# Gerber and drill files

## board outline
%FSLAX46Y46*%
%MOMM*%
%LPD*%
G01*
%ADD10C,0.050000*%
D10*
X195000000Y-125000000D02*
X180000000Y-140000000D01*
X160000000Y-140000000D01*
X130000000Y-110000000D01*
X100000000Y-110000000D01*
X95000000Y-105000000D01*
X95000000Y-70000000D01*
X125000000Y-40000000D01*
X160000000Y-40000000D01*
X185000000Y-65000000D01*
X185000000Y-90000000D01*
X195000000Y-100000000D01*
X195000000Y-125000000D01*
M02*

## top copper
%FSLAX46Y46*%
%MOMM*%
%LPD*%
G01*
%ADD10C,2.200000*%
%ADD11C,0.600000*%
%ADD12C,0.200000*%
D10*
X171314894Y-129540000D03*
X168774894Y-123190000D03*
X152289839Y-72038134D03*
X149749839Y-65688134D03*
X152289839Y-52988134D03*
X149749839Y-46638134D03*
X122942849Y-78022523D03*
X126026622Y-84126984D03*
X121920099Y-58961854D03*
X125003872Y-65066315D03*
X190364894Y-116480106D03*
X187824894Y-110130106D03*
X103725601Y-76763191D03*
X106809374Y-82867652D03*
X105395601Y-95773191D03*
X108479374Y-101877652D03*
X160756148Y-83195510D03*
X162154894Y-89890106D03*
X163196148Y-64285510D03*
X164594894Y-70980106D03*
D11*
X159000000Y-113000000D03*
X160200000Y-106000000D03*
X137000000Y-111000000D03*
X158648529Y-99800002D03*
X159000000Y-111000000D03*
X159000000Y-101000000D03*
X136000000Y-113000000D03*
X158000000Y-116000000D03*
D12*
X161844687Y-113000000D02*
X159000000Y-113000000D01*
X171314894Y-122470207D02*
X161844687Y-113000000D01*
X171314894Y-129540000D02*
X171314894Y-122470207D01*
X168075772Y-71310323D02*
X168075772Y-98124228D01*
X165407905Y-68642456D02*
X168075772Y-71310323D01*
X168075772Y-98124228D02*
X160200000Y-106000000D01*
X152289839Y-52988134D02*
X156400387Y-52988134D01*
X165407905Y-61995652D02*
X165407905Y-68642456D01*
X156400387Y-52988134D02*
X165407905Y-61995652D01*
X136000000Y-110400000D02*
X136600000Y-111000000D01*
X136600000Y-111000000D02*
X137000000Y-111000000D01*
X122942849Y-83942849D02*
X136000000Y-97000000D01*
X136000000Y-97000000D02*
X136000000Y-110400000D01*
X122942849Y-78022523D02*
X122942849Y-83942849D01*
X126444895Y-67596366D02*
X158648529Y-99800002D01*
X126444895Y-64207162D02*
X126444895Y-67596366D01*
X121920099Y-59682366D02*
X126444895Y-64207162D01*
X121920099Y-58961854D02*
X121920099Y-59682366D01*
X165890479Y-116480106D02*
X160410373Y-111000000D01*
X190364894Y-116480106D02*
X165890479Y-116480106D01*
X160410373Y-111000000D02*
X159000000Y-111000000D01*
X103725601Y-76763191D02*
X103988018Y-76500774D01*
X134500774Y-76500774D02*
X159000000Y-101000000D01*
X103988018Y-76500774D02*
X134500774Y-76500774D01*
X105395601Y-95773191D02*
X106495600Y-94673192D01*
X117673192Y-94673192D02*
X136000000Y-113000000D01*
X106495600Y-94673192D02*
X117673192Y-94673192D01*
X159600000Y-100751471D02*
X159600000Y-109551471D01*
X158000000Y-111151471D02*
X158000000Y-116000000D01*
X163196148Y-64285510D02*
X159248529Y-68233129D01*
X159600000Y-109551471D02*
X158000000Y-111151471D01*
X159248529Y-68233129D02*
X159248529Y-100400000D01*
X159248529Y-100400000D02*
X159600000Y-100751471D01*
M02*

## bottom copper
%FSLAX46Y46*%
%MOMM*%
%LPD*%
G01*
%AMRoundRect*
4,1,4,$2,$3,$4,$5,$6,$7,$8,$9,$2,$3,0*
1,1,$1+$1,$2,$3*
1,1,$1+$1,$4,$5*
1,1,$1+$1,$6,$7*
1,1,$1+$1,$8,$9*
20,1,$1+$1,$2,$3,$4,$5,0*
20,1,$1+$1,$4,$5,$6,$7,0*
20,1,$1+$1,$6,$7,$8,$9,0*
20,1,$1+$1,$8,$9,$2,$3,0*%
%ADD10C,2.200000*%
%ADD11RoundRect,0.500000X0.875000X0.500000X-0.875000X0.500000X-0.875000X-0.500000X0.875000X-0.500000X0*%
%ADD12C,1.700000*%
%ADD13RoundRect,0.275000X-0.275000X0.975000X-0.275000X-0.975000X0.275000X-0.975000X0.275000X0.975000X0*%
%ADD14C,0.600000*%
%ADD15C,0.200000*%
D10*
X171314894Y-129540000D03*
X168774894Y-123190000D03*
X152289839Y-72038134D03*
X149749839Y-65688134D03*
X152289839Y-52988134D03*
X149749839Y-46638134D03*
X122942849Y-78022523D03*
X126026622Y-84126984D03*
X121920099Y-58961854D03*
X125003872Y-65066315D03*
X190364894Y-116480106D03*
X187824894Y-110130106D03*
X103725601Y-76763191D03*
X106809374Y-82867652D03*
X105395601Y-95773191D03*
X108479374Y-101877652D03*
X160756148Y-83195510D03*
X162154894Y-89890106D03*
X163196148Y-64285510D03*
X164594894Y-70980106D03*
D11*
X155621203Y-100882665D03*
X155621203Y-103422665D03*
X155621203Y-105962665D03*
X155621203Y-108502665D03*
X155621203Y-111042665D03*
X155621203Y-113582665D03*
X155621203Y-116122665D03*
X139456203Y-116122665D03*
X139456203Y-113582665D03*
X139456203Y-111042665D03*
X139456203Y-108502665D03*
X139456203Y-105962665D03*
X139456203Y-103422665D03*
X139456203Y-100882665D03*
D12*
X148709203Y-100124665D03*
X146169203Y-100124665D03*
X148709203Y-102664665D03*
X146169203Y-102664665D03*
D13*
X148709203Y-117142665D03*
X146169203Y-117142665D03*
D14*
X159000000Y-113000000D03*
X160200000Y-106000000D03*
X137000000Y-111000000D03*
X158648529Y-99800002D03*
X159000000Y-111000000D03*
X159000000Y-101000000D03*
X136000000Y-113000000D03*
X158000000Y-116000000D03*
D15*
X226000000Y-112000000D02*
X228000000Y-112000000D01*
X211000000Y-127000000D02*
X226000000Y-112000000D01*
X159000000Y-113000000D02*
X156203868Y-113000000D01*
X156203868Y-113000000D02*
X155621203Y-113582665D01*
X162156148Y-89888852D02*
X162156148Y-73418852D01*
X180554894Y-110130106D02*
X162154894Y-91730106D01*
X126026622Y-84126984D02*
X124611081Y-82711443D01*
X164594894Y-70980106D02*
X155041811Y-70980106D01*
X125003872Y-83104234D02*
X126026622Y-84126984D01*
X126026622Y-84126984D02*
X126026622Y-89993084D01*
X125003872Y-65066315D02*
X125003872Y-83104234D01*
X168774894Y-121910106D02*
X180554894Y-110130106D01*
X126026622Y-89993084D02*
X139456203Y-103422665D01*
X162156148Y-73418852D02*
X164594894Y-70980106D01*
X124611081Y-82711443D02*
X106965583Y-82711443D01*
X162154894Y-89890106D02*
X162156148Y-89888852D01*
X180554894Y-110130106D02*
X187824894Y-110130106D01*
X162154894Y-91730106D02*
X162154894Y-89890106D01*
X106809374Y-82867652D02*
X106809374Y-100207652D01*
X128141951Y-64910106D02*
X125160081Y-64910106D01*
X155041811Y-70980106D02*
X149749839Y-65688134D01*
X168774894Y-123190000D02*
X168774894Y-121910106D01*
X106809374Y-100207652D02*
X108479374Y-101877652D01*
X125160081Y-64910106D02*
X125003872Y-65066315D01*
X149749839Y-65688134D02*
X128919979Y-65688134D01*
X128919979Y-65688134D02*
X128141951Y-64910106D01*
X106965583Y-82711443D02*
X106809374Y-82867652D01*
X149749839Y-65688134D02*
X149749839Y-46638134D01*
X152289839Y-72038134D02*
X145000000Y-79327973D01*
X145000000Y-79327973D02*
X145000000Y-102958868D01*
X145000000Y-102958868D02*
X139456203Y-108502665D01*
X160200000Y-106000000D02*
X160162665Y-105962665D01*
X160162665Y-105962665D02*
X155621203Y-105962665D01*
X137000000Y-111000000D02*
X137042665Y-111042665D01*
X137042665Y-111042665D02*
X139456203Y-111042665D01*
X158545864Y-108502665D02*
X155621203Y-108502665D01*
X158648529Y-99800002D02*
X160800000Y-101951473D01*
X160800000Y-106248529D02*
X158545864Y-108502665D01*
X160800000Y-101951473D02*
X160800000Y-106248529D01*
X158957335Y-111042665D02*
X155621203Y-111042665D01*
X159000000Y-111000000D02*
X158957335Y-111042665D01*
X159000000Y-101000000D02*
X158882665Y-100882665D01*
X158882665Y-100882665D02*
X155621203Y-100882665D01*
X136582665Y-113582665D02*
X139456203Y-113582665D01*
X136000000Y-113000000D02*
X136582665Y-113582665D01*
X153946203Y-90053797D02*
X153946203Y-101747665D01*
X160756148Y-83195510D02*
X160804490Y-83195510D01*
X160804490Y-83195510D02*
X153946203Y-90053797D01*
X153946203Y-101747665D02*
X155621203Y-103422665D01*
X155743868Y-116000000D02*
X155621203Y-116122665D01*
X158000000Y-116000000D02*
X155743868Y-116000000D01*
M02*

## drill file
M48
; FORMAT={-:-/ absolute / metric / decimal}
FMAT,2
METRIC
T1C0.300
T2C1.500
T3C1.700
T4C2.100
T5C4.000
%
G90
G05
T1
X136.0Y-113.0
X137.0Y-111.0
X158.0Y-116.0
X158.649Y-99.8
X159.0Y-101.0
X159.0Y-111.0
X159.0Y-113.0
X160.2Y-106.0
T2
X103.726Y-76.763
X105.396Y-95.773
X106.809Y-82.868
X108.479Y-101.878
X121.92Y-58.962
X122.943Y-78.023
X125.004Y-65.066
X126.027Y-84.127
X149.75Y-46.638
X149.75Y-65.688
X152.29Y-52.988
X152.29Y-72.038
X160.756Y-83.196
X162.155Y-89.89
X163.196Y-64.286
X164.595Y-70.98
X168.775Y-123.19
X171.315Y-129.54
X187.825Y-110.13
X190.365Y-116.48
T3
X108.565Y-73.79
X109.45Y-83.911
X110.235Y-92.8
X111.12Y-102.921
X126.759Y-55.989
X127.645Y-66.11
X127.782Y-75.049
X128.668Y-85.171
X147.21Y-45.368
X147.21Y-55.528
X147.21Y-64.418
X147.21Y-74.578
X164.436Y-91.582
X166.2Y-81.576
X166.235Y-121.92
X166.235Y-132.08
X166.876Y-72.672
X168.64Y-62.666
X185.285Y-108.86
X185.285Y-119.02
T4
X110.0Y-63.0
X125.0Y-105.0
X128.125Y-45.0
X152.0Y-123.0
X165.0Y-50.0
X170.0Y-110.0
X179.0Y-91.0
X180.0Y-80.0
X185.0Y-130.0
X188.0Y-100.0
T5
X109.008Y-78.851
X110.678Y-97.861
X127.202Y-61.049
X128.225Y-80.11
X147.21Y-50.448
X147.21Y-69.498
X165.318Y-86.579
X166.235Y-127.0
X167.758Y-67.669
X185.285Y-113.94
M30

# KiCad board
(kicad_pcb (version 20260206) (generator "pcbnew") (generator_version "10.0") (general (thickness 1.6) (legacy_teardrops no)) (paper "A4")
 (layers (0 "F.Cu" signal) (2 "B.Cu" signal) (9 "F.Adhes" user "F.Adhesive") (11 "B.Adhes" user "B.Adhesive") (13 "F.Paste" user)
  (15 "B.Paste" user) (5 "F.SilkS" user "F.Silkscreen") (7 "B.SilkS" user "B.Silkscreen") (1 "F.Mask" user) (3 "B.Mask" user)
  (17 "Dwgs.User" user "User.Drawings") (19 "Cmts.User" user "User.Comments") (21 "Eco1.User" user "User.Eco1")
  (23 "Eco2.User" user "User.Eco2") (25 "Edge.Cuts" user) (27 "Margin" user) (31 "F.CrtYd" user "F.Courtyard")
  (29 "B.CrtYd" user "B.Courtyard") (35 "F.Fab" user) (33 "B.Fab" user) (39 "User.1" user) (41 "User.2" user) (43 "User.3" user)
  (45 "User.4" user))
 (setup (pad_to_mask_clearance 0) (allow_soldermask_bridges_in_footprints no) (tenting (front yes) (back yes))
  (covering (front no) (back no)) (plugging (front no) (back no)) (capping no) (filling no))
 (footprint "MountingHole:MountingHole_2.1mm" (layer "F.Cu") (at 185 130)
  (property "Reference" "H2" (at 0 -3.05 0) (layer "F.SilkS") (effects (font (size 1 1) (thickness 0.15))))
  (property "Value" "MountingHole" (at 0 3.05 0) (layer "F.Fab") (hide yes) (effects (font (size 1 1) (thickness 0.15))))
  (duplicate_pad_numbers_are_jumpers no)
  (pad "" np_thru_hole circle (at 0 0) (size 2.1 2.1) (drill 2.1) (layers "*.Cu" "*.Mask")))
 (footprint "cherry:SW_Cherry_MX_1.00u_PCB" (layer "F.Cu") (at 171.314894 129.54 -90)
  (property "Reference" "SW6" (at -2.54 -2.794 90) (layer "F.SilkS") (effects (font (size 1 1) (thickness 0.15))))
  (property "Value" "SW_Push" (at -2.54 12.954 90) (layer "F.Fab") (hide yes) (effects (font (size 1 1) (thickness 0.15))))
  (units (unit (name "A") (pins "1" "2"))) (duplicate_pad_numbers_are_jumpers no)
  (pad "" np_thru_hole circle (at -7.62 5.08 270) (size 1.7 1.7) (drill 1.7) (layers "*.Cu" "*.Mask"))
  (pad "" np_thru_hole circle (at -2.54 5.08 270) (size 4 4) (drill 4) (layers "*.Cu" "*.Mask"))
  (pad "" np_thru_hole circle (at 2.54 5.08 270) (size 1.7 1.7) (drill 1.7) (layers "*.Cu" "*.Mask"))
  (pad "1" thru_hole circle (at 0 0 270) (size 2.2 2.2) (drill 1.5) (layers "*.Cu" "*.Mask") (remove_unused_layers no) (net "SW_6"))
  (pad "2" thru_hole circle (at -6.35 2.54 270) (size 2.2 2.2) (drill 1.5) (layers "*.Cu" "*.Mask") (remove_unused_layers no) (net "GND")))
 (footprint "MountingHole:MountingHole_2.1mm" (layer "F.Cu") (at 128.125 45)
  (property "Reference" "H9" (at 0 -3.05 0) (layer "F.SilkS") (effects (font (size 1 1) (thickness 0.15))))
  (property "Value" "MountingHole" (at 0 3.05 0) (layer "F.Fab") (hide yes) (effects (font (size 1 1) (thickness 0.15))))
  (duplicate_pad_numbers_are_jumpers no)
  (pad "" np_thru_hole circle (at 0 0) (size 2.1 2.1) (drill 2.1) (layers "*.Cu" "*.Mask")))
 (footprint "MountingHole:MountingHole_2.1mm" (layer "F.Cu") (at 170 110)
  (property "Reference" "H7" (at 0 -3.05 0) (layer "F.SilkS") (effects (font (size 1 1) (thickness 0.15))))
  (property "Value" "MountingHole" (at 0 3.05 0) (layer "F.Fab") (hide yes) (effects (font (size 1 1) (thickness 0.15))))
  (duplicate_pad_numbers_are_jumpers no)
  (pad "" np_thru_hole circle (at 0 0) (size 2.1 2.1) (drill 2.1) (layers "*.Cu" "*.Mask")))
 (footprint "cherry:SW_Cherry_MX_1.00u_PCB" (layer "F.Cu") (at 152.289839 72.038134 -90)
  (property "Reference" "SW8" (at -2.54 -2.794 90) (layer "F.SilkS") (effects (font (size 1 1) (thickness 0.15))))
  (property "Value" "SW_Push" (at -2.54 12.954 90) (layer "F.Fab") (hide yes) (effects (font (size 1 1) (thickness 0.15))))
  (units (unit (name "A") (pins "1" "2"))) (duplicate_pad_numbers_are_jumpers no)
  (pad "" np_thru_hole circle (at -7.62 5.08 270) (size 1.7 1.7) (drill 1.7) (layers "*.Cu" "*.Mask"))
  (pad "" np_thru_hole circle (at -2.54 5.08 270) (size 4 4) (drill 4) (layers "*.Cu" "*.Mask"))
  (pad "" np_thru_hole circle (at 2.54 5.08 270) (size 1.7 1.7) (drill 1.7) (layers "*.Cu" "*.Mask"))
  (pad "1" thru_hole circle (at 0 0 270) (size 2.2 2.2) (drill 1.5) (layers "*.Cu" "*.Mask") (remove_unused_layers no) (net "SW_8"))
  (pad "2" thru_hole circle (at -6.35 2.54 270) (size 2.2 2.2) (drill 1.5) (layers "*.Cu" "*.Mask") (remove_unused_layers no) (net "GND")))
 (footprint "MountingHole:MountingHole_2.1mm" (layer "F.Cu") (at 179 91)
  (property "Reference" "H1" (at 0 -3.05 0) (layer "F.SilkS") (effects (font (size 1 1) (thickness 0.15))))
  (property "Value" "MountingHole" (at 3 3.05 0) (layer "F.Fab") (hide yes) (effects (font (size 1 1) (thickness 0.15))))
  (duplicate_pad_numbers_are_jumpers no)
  (pad "" np_thru_hole circle (at 0 0) (size 2.1 2.1) (drill 2.1) (layers "*.Cu" "*.Mask")))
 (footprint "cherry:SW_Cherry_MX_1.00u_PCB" (layer "F.Cu") (at 152.289839 52.988134 -90)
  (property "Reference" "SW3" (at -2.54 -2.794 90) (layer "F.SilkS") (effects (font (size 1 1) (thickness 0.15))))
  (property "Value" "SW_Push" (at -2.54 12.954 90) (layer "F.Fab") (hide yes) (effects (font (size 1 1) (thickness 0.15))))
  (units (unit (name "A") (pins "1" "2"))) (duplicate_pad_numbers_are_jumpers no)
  (pad "" np_thru_hole circle (at -7.62 5.08 270) (size 1.7 1.7) (drill 1.7) (layers "*.Cu" "*.Mask"))
  (pad "" np_thru_hole circle (at -2.54 5.08 270) (size 4 4) (drill 4) (layers "*.Cu" "*.Mask"))
  (pad "" np_thru_hole circle (at 2.54 5.08 270) (size 1.7 1.7) (drill 1.7) (layers "*.Cu" "*.Mask"))
  (pad "1" thru_hole circle (at 0 0 270) (size 2.2 2.2) (drill 1.5) (layers "*.Cu" "*.Mask") (remove_unused_layers no) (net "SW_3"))
  (pad "2" thru_hole circle (at -6.35 2.54 270) (size 2.2 2.2) (drill 1.5) (layers "*.Cu" "*.Mask") (remove_unused_layers no) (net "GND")))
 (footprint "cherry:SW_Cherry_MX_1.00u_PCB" (layer "F.Cu") (at 122.942849 78.022523 95)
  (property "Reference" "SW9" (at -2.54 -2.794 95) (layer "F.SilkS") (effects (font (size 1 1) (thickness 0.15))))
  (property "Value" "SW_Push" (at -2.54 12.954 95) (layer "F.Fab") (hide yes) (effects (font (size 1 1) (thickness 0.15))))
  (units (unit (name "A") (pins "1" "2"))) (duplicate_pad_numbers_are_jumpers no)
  (pad "" np_thru_hole circle (at -7.62 5.08 95) (size 1.7 1.7) (drill 1.7) (layers "*.Cu" "*.Mask"))
  (pad "" np_thru_hole circle (at -2.54 5.08 95) (size 4 4) (drill 4) (layers "*.Cu" "*.Mask"))
  (pad "" np_thru_hole circle (at 2.54 5.08 95) (size 1.7 1.7) (drill 1.7) (layers "*.Cu" "*.Mask"))
  (pad "1" thru_hole circle (at 0 0 95) (size 2.2 2.2) (drill 1.5) (layers "*.Cu" "*.Mask") (remove_unused_layers no) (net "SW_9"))
  (pad "2" thru_hole circle (at -6.35 2.539999 95) (size 2.2 2.2) (drill 1.5) (layers "*.Cu" "*.Mask") (remove_unused_layers no) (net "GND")))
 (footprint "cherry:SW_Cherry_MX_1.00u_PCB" (layer "F.Cu") (at 121.920099 58.961854 95)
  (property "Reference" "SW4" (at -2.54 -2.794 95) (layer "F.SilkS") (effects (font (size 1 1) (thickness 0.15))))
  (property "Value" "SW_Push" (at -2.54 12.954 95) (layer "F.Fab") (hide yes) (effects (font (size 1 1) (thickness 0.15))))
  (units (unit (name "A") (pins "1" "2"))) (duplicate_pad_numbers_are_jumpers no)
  (pad "" np_thru_hole circle (at -7.62 5.08 95) (size 1.7 1.7) (drill 1.7) (layers "*.Cu" "*.Mask"))
  (pad "" np_thru_hole circle (at -2.54 5.08 95) (size 4 4) (drill 4) (layers "*.Cu" "*.Mask"))
  (pad "" np_thru_hole circle (at 2.54 5.08 95) (size 1.7 1.7) (drill 1.7) (layers "*.Cu" "*.Mask"))
  (pad "1" thru_hole circle (at 0 0 95) (size 2.2 2.2) (drill 1.5) (layers "*.Cu" "*.Mask") (remove_unused_layers no) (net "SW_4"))
  (pad "2" thru_hole circle (at -6.35 2.539999 95) (size 2.2 2.2) (drill 1.5) (layers "*.Cu" "*.Mask") (remove_unused_layers no) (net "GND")))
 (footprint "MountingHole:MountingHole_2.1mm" (layer "F.Cu") (at 110 63)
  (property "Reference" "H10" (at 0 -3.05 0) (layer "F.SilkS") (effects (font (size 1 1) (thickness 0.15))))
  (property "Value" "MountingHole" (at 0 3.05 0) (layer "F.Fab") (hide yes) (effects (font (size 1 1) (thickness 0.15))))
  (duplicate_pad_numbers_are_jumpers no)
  (pad "" np_thru_hole circle (at 0 0) (size 2.1 2.1) (drill 2.1) (layers "*.Cu" "*.Mask")))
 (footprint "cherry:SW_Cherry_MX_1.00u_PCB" (layer "F.Cu") (at 190.364894 116.480106 -90)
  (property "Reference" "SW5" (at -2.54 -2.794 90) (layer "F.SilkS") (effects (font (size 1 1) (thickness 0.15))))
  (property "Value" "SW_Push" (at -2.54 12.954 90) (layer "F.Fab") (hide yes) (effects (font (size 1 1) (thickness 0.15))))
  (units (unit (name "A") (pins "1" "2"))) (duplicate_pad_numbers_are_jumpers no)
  (pad "" np_thru_hole circle (at -7.62 5.08 270) (size 1.7 1.7) (drill 1.7) (layers "*.Cu" "*.Mask"))
  (pad "" np_thru_hole circle (at -2.54 5.08 270) (size 4 4) (drill 4) (layers "*.Cu" "*.Mask"))
  (pad "" np_thru_hole circle (at 2.54 5.08 270) (size 1.7 1.7) (drill 1.7) (layers "*.Cu" "*.Mask"))
  (pad "1" thru_hole circle (at 0 0 270) (size 2.2 2.2) (drill 1.5) (layers "*.Cu" "*.Mask") (remove_unused_layers no) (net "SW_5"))
  (pad "2" thru_hole circle (at -6.35 2.54 270) (size 2.2 2.2) (drill 1.5) (layers "*.Cu" "*.Mask") (remove_unused_layers no) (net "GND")))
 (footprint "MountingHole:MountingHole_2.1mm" (layer "F.Cu") (at 125 105)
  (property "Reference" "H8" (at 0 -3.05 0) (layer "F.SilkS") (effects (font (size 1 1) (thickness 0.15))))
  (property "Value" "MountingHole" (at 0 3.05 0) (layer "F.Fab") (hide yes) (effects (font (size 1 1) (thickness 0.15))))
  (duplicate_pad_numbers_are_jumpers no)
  (pad "" np_thru_hole circle (at 0 0) (size 2.1 2.1) (drill 2.1) (layers "*.Cu" "*.Mask")))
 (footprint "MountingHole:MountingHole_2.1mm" (layer "F.Cu") (at 188 100)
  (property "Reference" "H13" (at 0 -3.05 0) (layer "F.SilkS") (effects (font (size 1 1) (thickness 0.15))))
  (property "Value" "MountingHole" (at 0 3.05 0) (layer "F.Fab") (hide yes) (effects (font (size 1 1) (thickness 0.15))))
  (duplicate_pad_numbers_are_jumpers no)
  (pad "" np_thru_hole circle (at 0 0) (size 2.1 2.1) (drill 2.1) (layers "*.Cu" "*.Mask")))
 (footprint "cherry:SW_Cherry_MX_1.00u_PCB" (layer "F.Cu") (at 103.725601 76.763191 95)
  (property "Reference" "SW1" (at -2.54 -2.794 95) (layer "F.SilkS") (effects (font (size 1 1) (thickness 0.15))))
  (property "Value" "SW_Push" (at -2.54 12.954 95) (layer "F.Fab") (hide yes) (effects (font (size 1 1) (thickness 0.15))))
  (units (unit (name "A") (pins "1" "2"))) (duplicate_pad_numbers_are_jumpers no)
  (pad "" np_thru_hole circle (at -7.62 5.08 95) (size 1.7 1.7) (drill 1.7) (layers "*.Cu" "*.Mask"))
  (pad "" np_thru_hole circle (at -2.54 5.08 95) (size 4 4) (drill 4) (layers "*.Cu" "*.Mask"))
  (pad "" np_thru_hole circle (at 2.54 5.08 95) (size 1.7 1.7) (drill 1.7) (layers "*.Cu" "*.Mask"))
  (pad "1" thru_hole circle (at 0 0 95) (size 2.2 2.2) (drill 1.5) (layers "*.Cu" "*.Mask") (remove_unused_layers no) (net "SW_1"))
  (pad "2" thru_hole circle (at -6.35 2.539999 95) (size 2.2 2.2) (drill 1.5) (layers "*.Cu" "*.Mask") (remove_unused_layers no) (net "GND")))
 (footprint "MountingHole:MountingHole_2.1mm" (layer "F.Cu") (at 165 50)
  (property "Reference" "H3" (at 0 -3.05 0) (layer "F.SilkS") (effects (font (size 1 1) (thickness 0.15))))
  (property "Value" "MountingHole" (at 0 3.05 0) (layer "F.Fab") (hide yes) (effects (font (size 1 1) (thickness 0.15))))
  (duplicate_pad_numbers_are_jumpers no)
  (pad "" np_thru_hole circle (at 0 0) (size 2.1 2.1) (drill 2.1) (layers "*.Cu" "*.Mask")))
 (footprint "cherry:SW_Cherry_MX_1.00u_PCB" (layer "F.Cu") (at 105.395601 95.773191 95)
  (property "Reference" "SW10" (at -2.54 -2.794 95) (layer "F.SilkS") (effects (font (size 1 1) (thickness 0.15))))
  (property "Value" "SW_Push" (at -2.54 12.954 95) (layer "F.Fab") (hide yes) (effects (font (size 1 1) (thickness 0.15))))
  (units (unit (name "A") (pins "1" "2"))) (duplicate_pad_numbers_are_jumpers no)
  (pad "" np_thru_hole circle (at -7.62 5.08 95) (size 1.7 1.7) (drill 1.7) (layers "*.Cu" "*.Mask"))
  (pad "" np_thru_hole circle (at -2.54 5.08 95) (size 4 4) (drill 4) (layers "*.Cu" "*.Mask"))
  (pad "" np_thru_hole circle (at 2.54 5.08 95) (size 1.7 1.7) (drill 1.7) (layers "*.Cu" "*.Mask"))
  (pad "1" thru_hole circle (at 0 0 95) (size 2.2 2.2) (drill 1.5) (layers "*.Cu" "*.Mask") (remove_unused_layers no) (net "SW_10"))
  (pad "2" thru_hole circle (at -6.35 2.539999 95) (size 2.2 2.2) (drill 1.5) (layers "*.Cu" "*.Mask") (remove_unused_layers no) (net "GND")))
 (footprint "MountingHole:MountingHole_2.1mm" (layer "F.Cu") (at 180 80)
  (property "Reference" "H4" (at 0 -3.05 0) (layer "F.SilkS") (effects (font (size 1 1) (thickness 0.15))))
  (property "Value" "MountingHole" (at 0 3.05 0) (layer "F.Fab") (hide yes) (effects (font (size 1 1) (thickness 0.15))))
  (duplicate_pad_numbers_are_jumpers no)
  (pad "" np_thru_hole circle (at 0 0) (size 2.1 2.1) (drill 2.1) (layers "*.Cu" "*.Mask")))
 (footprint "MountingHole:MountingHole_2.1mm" (layer "F.Cu") (at 152 123)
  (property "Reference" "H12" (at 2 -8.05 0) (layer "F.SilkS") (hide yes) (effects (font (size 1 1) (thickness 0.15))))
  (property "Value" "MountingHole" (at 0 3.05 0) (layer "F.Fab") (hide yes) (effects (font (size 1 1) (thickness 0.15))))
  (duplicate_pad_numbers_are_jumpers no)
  (pad "" np_thru_hole circle (at 0 0) (size 2.1 2.1) (drill 2.1) (layers "*.Cu" "*.Mask")))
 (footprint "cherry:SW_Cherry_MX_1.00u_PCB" (layer "F.Cu") (at 160.756148 83.19551 80)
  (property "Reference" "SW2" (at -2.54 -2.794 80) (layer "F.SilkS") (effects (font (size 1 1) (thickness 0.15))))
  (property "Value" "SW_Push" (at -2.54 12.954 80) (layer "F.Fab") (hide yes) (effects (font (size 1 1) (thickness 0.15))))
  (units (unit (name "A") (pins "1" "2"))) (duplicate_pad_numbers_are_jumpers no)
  (pad "" np_thru_hole circle (at -7.62 5.08 80) (size 1.7 1.7) (drill 1.7) (layers "*.Cu" "*.Mask"))
  (pad "" np_thru_hole circle (at -2.54 5.08 80) (size 4 4) (drill 4) (layers "*.Cu" "*.Mask"))
  (pad "" np_thru_hole circle (at 2.54 5.08 80) (size 1.7 1.7) (drill 1.7) (layers "*.Cu" "*.Mask"))
  (pad "1" thru_hole circle (at 0 0 80) (size 2.2 2.2) (drill 1.5) (layers "*.Cu" "*.Mask") (remove_unused_layers no) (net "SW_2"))
  (pad "2" thru_hole circle (at -6.35 2.54 80) (size 2.2 2.2) (drill 1.5) (layers "*.Cu" "*.Mask") (remove_unused_layers no) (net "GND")))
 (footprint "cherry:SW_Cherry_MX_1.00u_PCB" (layer "F.Cu") (at 163.196148 64.28551 80)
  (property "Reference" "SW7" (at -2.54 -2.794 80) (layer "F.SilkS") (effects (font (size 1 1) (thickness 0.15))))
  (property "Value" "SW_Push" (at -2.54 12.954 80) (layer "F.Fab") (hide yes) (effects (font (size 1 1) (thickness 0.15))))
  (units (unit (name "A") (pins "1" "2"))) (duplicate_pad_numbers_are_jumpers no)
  (pad "" np_thru_hole circle (at -7.62 5.08 80) (size 1.7 1.7) (drill 1.7) (layers "*.Cu" "*.Mask"))
  (pad "" np_thru_hole circle (at -2.54 5.08 80) (size 4 4) (drill 4) (layers "*.Cu" "*.Mask"))
  (pad "" np_thru_hole circle (at 2.54 5.08 80) (size 1.7 1.7) (drill 1.7) (layers "*.Cu" "*.Mask"))
  (pad "1" thru_hole circle (at 0 0 80) (size 2.2 2.2) (drill 1.5) (layers "*.Cu" "*.Mask") (remove_unused_layers no) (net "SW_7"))
  (pad "2" thru_hole circle (at -6.35 2.54 80) (size 2.2 2.2) (drill 1.5) (layers "*.Cu" "*.Mask") (remove_unused_layers no) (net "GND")))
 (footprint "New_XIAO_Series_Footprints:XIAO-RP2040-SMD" (layer "B.Cu") (at 156.456203 119.002665 180)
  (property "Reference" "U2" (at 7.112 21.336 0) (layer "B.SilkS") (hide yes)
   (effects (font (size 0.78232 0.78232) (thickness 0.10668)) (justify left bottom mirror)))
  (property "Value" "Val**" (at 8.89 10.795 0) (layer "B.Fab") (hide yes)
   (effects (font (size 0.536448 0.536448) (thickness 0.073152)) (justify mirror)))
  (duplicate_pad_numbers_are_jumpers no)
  (pad "1" smd roundrect (at 0.835 18.12 180) (size 2.75 2) (layers "B.Cu" "B.Mask" "B.Paste") (roundrect_rratio 0.25) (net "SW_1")
   (solder_mask_margin 0.0508) (thermal_bridge_angle 45))
  (pad "2" smd roundrect (at 0.835 15.58 180) (size 2.75 2) (layers "B.Cu" "B.Mask" "B.Paste") (roundrect_rratio 0.25) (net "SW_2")
   (solder_mask_margin 0.0508) (thermal_bridge_angle 45))
  (pad "3" smd roundrect (at 0.835 13.04 180) (size 2.75 2) (layers "B.Cu" "B.Mask" "B.Paste") (roundrect_rratio 0.25) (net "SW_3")
   (solder_mask_margin 0.0508) (thermal_bridge_angle 45))
  (pad "4" smd roundrect (at 0.835 10.5 180) (size 2.75 2) (layers "B.Cu" "B.Mask" "B.Paste") (roundrect_rratio 0.25) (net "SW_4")
   (solder_mask_margin 0.0508) (thermal_bridge_angle 45))
  (pad "5" smd roundrect (at 0.835 7.96 180) (size 2.75 2) (layers "B.Cu" "B.Mask" "B.Paste") (roundrect_rratio 0.25) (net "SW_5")
   (solder_mask_margin 0.0508) (thermal_bridge_angle 45))
  (pad "6" smd roundrect (at 0.835 5.42 180) (size 2.75 2) (layers "B.Cu" "B.Mask" "B.Paste") (roundrect_rratio 0.25) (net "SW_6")
   (solder_mask_margin 0.0508) (thermal_bridge_angle 45))
  (pad "7" smd roundrect (at 0.835 2.88 180) (size 2.75 2) (layers "B.Cu" "B.Mask" "B.Paste") (roundrect_rratio 0.25) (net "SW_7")
   (solder_mask_margin 0.0508) (thermal_bridge_angle 45))
  (pad "8" smd roundrect (at 17 2.88 180) (size 2.75 2) (layers "B.Cu" "B.Mask" "B.Paste") (roundrect_rratio 0.25)
   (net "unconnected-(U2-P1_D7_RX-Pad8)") (solder_mask_margin 0.0508) (thermal_bridge_angle 45))
  (pad "9" smd roundrect (at 17 5.42 180) (size 2.75 2) (layers "B.Cu" "B.Mask" "B.Paste") (roundrect_rratio 0.25) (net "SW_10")
   (solder_mask_margin 0.0508) (thermal_bridge_angle 45))
  (pad "10" smd roundrect (at 17 7.96 180) (size 2.75 2) (layers "B.Cu" "B.Mask" "B.Paste") (roundrect_rratio 0.25) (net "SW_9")
   (solder_mask_margin 0.0508) (thermal_bridge_angle 45))
  (pad "11" smd roundrect (at 17 10.5 180) (size 2.75 2) (layers "B.Cu" "B.Mask" "B.Paste") (roundrect_rratio 0.25) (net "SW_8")
   (solder_mask_margin 0.0508) (thermal_bridge_angle 45))
  (pad "12" smd roundrect (at 17 13.04 180) (size 2.75 2) (layers "B.Cu" "B.Mask" "B.Paste") (roundrect_rratio 0.25)
   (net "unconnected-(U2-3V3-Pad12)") (solder_mask_margin 0.0508) (thermal_bridge_angle 45))
  (pad "13" smd roundrect (at 17 15.58 180) (size 2.75 2) (layers "B.Cu" "B.Mask" "B.Paste") (roundrect_rratio 0.25) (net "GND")
   (solder_mask_margin 0.0508) (thermal_bridge_angle 45))
  (pad "14" smd roundrect (at 17 18.12 180) (size 2.75 2) (layers "B.Cu" "B.Mask" "B.Paste") (roundrect_rratio 0.25)
   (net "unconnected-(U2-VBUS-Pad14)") (solder_mask_margin 0.0508) (thermal_bridge_angle 45))
  (pad "24" smd circle (at 7.747 18.878 180) (size 1.7 1.7) (layers "B.Cu" "B.Mask" "B.Paste") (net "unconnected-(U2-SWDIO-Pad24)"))
  (pad "25" smd circle (at 10.287 18.878 180) (size 1.7 1.7) (layers "B.Cu" "B.Mask" "B.Paste") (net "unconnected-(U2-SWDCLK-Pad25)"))
  (pad "26" smd circle (at 7.747 16.338 180) (size 1.7 1.7) (layers "B.Cu" "B.Mask" "B.Paste") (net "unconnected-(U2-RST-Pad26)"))
  (pad "27" smd circle (at 10.287 16.338 180) (size 1.7 1.7) (layers "B.Cu" "B.Mask" "B.Paste") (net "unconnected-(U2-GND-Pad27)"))
  (pad "32" smd roundrect (at 7.747 1.86 270) (size 2.5 1.1) (layers "B.Cu" "B.Mask" "B.Paste") (roundrect_rratio 0.25)
   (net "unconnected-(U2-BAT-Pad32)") (thermal_bridge_angle 45))
  (pad "33" smd roundrect (at 10.287 1.86 270) (size 2.5 1.1) (layers "B.Cu" "B.Mask" "B.Paste") (roundrect_rratio 0.25)
   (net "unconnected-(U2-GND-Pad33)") (thermal_bridge_angle 45)))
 (gr_poly
  (pts (xy 195 125) (xy 180 140) (xy 160 140) (xy 130 110) (xy 100 110) (xy 95 105) (xy 95 70) (xy 125 40) (xy 160 40) (xy 185 65)
   (xy 185 90) (xy 195 100))
  (stroke (width 0.05) (type solid)) (fill no) (layer "Edge.Cuts"))
 (segment (start 226 112) (end 228 112) (width 0.2) (layer "B.Cu") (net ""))
 (segment (start 211 127) (end 226 112) (width 0.2) (layer "B.Cu") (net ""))
 (segment (start 161.844687 113) (end 159 113) (width 0.2) (layer "F.Cu") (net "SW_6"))
 (segment (start 171.314894 122.470207) (end 161.844687 113) (width 0.2) (layer "F.Cu") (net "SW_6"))
 (segment (start 171.314894 129.54) (end 171.314894 122.470207) (width 0.2) (layer "F.Cu") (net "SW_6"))
 (via (at 159 113) (size 0.6) (drill 0.3) (layers "F.Cu" "B.Cu") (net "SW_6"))
 (segment (start 159 113) (end 156.203868 113) (width 0.2) (layer "B.Cu") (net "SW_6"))
 (segment (start 156.203868 113) (end 155.621203 113.582665) (width 0.2) (layer "B.Cu") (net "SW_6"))
 (segment (start 162.156148 89.888852) (end 162.156148 73.418852) (width 0.2) (layer "B.Cu") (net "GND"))
 (segment (start 180.554894 110.130106) (end 162.154894 91.730106) (width 0.2) (layer "B.Cu") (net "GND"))
 (segment (start 126.026622 84.126984) (end 124.611081 82.711443) (width 0.2) (layer "B.Cu") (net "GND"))
 (segment (start 164.594894 70.980106) (end 155.041811 70.980106) (width 0.2) (layer "B.Cu") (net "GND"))
 (segment (start 125.003872 83.104234) (end 126.026622 84.126984) (width 0.2) (layer "B.Cu") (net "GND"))
 (segment (start 126.026622 84.126984) (end 126.026622 89.993084) (width 0.2) (layer "B.Cu") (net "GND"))
 (segment (start 125.003872 65.066315) (end 125.003872 83.104234) (width 0.2) (layer "B.Cu") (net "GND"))
 (segment (start 168.774894 121.910106) (end 180.554894 110.130106) (width 0.2) (layer "B.Cu") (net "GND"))
 (segment (start 126.026622 89.993084) (end 139.456203 103.422665) (width 0.2) (layer "B.Cu") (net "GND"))
 (segment (start 162.156148 73.418852) (end 164.594894 70.980106) (width 0.2) (layer "B.Cu") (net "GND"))
 (segment (start 124.611081 82.711443) (end 106.965583 82.711443) (width 0.2) (layer "B.Cu") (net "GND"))
 (segment (start 162.154894 89.890106) (end 162.156148 89.888852) (width 0.2) (layer "B.Cu") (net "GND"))
 (segment (start 180.554894 110.130106) (end 187.824894 110.130106) (width 0.2) (layer "B.Cu") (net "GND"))
 (segment (start 162.154894 91.730106) (end 162.154894 89.890106) (width 0.2) (layer "B.Cu") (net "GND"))
 (segment (start 106.809374 82.867652) (end 106.809374 100.207652) (width 0.2) (layer "B.Cu") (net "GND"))
 (segment (start 128.141951 64.910106) (end 125.160081 64.910106) (width 0.2) (layer "B.Cu") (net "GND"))
 (segment (start 155.041811 70.980106) (end 149.749839 65.688134) (width 0.2) (layer "B.Cu") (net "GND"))
 (segment (start 168.774894 123.19) (end 168.774894 121.910106) (width 0.2) (layer "B.Cu") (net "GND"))
 (segment (start 106.809374 100.207652) (end 108.479374 101.877652) (width 0.2) (layer "B.Cu") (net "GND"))
 (segment (start 125.160081 64.910106) (end 125.003872 65.066315) (width 0.2) (layer "B.Cu") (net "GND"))
 (segment (start 149.749839 65.688134) (end 128.919979 65.688134) (width 0.2) (layer "B.Cu") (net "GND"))
 (segment (start 128.919979 65.688134) (end 128.141951 64.910106) (width 0.2) (layer "B.Cu") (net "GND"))
 (segment (start 106.965583 82.711443) (end 106.809374 82.867652) (width 0.2) (layer "B.Cu") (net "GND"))
 (segment (start 149.749839 65.688134) (end 149.749839 46.638134) (width 0.2) (layer "B.Cu") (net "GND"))
 (segment (start 152.289839 72.038134) (end 145 79.327973) (width 0.2) (layer "B.Cu") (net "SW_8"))
 (segment (start 145 79.327973) (end 145 102.958868) (width 0.2) (layer "B.Cu") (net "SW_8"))
 (segment (start 145 102.958868) (end 139.456203 108.502665) (width 0.2) (layer "B.Cu") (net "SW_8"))
 (segment (start 168.075772 71.310323) (end 168.075772 98.124228) (width 0.2) (layer "F.Cu") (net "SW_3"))
 (segment (start 165.407905 68.642456) (end 168.075772 71.310323) (width 0.2) (layer "F.Cu") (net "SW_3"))
 (segment (start 168.075772 98.124228) (end 160.2 106) (width 0.2) (layer "F.Cu") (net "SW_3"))
 (segment (start 152.289839 52.988134) (end 156.400387 52.988134) (width 0.2) (layer "F.Cu") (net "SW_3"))
 (segment (start 165.407905 61.995652) (end 165.407905 68.642456) (width 0.2) (layer "F.Cu") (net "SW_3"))
 (segment (start 156.400387 52.988134) (end 165.407905 61.995652) (width 0.2) (layer "F.Cu") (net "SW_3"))
 (via (at 160.2 106) (size 0.6) (drill 0.3) (layers "F.Cu" "B.Cu") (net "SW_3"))
 (segment (start 160.2 106) (end 160.162665 105.962665) (width 0.2) (layer "B.Cu") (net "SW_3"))
 (segment (start 160.162665 105.962665) (end 155.621203 105.962665) (width 0.2) (layer "B.Cu") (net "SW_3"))
 (segment (start 136 110.4) (end 136.6 111) (width 0.2) (layer "F.Cu") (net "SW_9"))
 (segment (start 136.6 111) (end 137 111) (width 0.2) (layer "F.Cu") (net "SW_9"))
 (segment (start 122.942849 83.942849) (end 136 97) (width 0.2) (layer "F.Cu") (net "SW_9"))
 (segment (start 136 97) (end 136 110.4) (width 0.2) (layer "F.Cu") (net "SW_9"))
 (segment (start 122.942849 78.022523) (end 122.942849 83.942849) (width 0.2) (layer "F.Cu") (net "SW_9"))
 (via (at 137 111) (size 0.6) (drill 0.3) (layers "F.Cu" "B.Cu") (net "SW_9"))
 (segment (start 137 111) (end 137.042665 111.042665) (width 0.2) (layer "B.Cu") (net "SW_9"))
 (segment (start 137.042665 111.042665) (end 139.456203 111.042665) (width 0.2) (layer "B.Cu") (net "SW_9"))
 (segment (start 126.444895 67.596366) (end 158.648529 99.800002) (width 0.2) (layer "F.Cu") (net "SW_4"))
 (segment (start 126.444895 64.207162) (end 126.444895 67.596366) (width 0.2) (layer "F.Cu") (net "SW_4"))
 (segment (start 121.920099 59.682366) (end 126.444895 64.207162) (width 0.2) (layer "F.Cu") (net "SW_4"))
 (segment (start 121.920099 58.961854) (end 121.920099 59.682366) (width 0.2) (layer "F.Cu") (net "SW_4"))
 (via (at 158.648529 99.800002) (size 0.6) (drill 0.3) (layers "F.Cu" "B.Cu") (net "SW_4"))
 (segment (start 158.545864 108.502665) (end 155.621203 108.502665) (width 0.2) (layer "B.Cu") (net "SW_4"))
 (segment (start 158.648529 99.800002) (end 160.8 101.951473) (width 0.2) (layer "B.Cu") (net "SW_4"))
 (segment (start 160.8 106.248529) (end 158.545864 108.502665) (width 0.2) (layer "B.Cu") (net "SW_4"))
 (segment (start 160.8 101.951473) (end 160.8 106.248529) (width 0.2) (layer "B.Cu") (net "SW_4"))
 (segment (start 165.890479 116.480106) (end 160.410373 111) (width 0.2) (layer "F.Cu") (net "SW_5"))
 (segment (start 190.364894 116.480106) (end 165.890479 116.480106) (width 0.2) (layer "F.Cu") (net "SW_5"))
 (segment (start 160.410373 111) (end 159 111) (width 0.2) (layer "F.Cu") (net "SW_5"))
 (via (at 159 111) (size 0.6) (drill 0.3) (layers "F.Cu" "B.Cu") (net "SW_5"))
 (segment (start 158.957335 111.042665) (end 155.621203 111.042665) (width 0.2) (layer "B.Cu") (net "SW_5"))
 (segment (start 159 111) (end 158.957335 111.042665) (width 0.2) (layer "B.Cu") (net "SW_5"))
 (segment (start 103.725601 76.763191) (end 103.988018 76.500774) (width 0.2) (layer "F.Cu") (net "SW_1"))
 (segment (start 134.500774 76.500774) (end 159 101) (width 0.2) (layer "F.Cu") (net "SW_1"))
 (segment (start 103.988018 76.500774) (end 134.500774 76.500774) (width 0.2) (layer "F.Cu") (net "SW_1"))
 (via (at 159 101) (size 0.6) (drill 0.3) (layers "F.Cu" "B.Cu") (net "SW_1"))
 (segment (start 159 101) (end 158.882665 100.882665) (width 0.2) (layer "B.Cu") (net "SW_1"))
 (segment (start 158.882665 100.882665) (end 155.621203 100.882665) (width 0.2) (layer "B.Cu") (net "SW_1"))
 (segment (start 105.395601 95.773191) (end 106.4956 94.673192) (width 0.2) (layer "F.Cu") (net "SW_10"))
 (segment (start 117.673192 94.673192) (end 136 113) (width 0.2) (layer "F.Cu") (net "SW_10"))
 (segment (start 106.4956 94.673192) (end 117.673192 94.673192) (width 0.2) (layer "F.Cu") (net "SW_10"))
 (via (at 136 113) (size 0.6) (drill 0.3) (layers "F.Cu" "B.Cu") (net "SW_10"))
 (segment (start 136.582665 113.582665) (end 139.456203 113.582665) (width 0.2) (layer "B.Cu") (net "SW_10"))
 (segment (start 136 113) (end 136.582665 113.582665) (width 0.2) (layer "B.Cu") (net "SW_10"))
 (segment (start 153.946203 90.053797) (end 153.946203 101.747665) (width 0.2) (layer "B.Cu") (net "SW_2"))
 (segment (start 160.756148 83.19551) (end 160.80449 83.19551) (width 0.2) (layer "B.Cu") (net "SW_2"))
 (segment (start 160.80449 83.19551) (end 153.946203 90.053797) (width 0.2) (layer "B.Cu") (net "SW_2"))
 (segment (start 153.946203 101.747665) (end 155.621203 103.422665) (width 0.2) (layer "B.Cu") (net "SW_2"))
 (segment (start 159.6 100.751471) (end 159.6 109.551471) (width 0.2) (layer "F.Cu") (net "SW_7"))
 (segment (start 158 111.151471) (end 158 116) (width 0.2) (layer "F.Cu") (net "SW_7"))
 (segment (start 163.196148 64.28551) (end 159.248529 68.233129) (width 0.2) (layer "F.Cu") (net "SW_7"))
 (segment (start 159.6 109.551471) (end 158 111.151471) (width 0.2) (layer "F.Cu") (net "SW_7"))
 (segment (start 159.248529 68.233129) (end 159.248529 100.4) (width 0.2) (layer "F.Cu") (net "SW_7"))
 (segment (start 159.248529 100.4) (end 159.6 100.751471) (width 0.2) (layer "F.Cu") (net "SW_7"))
 (via (at 158 116) (size 0.6) (drill 0.3) (layers "F.Cu" "B.Cu") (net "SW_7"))
 (segment (start 155.743868 116) (end 155.621203 116.122665) (width 0.2) (layer "B.Cu") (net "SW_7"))
 (segment (start 158 116) (end 155.743868 116) (width 0.2) (layer "B.Cu") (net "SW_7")))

